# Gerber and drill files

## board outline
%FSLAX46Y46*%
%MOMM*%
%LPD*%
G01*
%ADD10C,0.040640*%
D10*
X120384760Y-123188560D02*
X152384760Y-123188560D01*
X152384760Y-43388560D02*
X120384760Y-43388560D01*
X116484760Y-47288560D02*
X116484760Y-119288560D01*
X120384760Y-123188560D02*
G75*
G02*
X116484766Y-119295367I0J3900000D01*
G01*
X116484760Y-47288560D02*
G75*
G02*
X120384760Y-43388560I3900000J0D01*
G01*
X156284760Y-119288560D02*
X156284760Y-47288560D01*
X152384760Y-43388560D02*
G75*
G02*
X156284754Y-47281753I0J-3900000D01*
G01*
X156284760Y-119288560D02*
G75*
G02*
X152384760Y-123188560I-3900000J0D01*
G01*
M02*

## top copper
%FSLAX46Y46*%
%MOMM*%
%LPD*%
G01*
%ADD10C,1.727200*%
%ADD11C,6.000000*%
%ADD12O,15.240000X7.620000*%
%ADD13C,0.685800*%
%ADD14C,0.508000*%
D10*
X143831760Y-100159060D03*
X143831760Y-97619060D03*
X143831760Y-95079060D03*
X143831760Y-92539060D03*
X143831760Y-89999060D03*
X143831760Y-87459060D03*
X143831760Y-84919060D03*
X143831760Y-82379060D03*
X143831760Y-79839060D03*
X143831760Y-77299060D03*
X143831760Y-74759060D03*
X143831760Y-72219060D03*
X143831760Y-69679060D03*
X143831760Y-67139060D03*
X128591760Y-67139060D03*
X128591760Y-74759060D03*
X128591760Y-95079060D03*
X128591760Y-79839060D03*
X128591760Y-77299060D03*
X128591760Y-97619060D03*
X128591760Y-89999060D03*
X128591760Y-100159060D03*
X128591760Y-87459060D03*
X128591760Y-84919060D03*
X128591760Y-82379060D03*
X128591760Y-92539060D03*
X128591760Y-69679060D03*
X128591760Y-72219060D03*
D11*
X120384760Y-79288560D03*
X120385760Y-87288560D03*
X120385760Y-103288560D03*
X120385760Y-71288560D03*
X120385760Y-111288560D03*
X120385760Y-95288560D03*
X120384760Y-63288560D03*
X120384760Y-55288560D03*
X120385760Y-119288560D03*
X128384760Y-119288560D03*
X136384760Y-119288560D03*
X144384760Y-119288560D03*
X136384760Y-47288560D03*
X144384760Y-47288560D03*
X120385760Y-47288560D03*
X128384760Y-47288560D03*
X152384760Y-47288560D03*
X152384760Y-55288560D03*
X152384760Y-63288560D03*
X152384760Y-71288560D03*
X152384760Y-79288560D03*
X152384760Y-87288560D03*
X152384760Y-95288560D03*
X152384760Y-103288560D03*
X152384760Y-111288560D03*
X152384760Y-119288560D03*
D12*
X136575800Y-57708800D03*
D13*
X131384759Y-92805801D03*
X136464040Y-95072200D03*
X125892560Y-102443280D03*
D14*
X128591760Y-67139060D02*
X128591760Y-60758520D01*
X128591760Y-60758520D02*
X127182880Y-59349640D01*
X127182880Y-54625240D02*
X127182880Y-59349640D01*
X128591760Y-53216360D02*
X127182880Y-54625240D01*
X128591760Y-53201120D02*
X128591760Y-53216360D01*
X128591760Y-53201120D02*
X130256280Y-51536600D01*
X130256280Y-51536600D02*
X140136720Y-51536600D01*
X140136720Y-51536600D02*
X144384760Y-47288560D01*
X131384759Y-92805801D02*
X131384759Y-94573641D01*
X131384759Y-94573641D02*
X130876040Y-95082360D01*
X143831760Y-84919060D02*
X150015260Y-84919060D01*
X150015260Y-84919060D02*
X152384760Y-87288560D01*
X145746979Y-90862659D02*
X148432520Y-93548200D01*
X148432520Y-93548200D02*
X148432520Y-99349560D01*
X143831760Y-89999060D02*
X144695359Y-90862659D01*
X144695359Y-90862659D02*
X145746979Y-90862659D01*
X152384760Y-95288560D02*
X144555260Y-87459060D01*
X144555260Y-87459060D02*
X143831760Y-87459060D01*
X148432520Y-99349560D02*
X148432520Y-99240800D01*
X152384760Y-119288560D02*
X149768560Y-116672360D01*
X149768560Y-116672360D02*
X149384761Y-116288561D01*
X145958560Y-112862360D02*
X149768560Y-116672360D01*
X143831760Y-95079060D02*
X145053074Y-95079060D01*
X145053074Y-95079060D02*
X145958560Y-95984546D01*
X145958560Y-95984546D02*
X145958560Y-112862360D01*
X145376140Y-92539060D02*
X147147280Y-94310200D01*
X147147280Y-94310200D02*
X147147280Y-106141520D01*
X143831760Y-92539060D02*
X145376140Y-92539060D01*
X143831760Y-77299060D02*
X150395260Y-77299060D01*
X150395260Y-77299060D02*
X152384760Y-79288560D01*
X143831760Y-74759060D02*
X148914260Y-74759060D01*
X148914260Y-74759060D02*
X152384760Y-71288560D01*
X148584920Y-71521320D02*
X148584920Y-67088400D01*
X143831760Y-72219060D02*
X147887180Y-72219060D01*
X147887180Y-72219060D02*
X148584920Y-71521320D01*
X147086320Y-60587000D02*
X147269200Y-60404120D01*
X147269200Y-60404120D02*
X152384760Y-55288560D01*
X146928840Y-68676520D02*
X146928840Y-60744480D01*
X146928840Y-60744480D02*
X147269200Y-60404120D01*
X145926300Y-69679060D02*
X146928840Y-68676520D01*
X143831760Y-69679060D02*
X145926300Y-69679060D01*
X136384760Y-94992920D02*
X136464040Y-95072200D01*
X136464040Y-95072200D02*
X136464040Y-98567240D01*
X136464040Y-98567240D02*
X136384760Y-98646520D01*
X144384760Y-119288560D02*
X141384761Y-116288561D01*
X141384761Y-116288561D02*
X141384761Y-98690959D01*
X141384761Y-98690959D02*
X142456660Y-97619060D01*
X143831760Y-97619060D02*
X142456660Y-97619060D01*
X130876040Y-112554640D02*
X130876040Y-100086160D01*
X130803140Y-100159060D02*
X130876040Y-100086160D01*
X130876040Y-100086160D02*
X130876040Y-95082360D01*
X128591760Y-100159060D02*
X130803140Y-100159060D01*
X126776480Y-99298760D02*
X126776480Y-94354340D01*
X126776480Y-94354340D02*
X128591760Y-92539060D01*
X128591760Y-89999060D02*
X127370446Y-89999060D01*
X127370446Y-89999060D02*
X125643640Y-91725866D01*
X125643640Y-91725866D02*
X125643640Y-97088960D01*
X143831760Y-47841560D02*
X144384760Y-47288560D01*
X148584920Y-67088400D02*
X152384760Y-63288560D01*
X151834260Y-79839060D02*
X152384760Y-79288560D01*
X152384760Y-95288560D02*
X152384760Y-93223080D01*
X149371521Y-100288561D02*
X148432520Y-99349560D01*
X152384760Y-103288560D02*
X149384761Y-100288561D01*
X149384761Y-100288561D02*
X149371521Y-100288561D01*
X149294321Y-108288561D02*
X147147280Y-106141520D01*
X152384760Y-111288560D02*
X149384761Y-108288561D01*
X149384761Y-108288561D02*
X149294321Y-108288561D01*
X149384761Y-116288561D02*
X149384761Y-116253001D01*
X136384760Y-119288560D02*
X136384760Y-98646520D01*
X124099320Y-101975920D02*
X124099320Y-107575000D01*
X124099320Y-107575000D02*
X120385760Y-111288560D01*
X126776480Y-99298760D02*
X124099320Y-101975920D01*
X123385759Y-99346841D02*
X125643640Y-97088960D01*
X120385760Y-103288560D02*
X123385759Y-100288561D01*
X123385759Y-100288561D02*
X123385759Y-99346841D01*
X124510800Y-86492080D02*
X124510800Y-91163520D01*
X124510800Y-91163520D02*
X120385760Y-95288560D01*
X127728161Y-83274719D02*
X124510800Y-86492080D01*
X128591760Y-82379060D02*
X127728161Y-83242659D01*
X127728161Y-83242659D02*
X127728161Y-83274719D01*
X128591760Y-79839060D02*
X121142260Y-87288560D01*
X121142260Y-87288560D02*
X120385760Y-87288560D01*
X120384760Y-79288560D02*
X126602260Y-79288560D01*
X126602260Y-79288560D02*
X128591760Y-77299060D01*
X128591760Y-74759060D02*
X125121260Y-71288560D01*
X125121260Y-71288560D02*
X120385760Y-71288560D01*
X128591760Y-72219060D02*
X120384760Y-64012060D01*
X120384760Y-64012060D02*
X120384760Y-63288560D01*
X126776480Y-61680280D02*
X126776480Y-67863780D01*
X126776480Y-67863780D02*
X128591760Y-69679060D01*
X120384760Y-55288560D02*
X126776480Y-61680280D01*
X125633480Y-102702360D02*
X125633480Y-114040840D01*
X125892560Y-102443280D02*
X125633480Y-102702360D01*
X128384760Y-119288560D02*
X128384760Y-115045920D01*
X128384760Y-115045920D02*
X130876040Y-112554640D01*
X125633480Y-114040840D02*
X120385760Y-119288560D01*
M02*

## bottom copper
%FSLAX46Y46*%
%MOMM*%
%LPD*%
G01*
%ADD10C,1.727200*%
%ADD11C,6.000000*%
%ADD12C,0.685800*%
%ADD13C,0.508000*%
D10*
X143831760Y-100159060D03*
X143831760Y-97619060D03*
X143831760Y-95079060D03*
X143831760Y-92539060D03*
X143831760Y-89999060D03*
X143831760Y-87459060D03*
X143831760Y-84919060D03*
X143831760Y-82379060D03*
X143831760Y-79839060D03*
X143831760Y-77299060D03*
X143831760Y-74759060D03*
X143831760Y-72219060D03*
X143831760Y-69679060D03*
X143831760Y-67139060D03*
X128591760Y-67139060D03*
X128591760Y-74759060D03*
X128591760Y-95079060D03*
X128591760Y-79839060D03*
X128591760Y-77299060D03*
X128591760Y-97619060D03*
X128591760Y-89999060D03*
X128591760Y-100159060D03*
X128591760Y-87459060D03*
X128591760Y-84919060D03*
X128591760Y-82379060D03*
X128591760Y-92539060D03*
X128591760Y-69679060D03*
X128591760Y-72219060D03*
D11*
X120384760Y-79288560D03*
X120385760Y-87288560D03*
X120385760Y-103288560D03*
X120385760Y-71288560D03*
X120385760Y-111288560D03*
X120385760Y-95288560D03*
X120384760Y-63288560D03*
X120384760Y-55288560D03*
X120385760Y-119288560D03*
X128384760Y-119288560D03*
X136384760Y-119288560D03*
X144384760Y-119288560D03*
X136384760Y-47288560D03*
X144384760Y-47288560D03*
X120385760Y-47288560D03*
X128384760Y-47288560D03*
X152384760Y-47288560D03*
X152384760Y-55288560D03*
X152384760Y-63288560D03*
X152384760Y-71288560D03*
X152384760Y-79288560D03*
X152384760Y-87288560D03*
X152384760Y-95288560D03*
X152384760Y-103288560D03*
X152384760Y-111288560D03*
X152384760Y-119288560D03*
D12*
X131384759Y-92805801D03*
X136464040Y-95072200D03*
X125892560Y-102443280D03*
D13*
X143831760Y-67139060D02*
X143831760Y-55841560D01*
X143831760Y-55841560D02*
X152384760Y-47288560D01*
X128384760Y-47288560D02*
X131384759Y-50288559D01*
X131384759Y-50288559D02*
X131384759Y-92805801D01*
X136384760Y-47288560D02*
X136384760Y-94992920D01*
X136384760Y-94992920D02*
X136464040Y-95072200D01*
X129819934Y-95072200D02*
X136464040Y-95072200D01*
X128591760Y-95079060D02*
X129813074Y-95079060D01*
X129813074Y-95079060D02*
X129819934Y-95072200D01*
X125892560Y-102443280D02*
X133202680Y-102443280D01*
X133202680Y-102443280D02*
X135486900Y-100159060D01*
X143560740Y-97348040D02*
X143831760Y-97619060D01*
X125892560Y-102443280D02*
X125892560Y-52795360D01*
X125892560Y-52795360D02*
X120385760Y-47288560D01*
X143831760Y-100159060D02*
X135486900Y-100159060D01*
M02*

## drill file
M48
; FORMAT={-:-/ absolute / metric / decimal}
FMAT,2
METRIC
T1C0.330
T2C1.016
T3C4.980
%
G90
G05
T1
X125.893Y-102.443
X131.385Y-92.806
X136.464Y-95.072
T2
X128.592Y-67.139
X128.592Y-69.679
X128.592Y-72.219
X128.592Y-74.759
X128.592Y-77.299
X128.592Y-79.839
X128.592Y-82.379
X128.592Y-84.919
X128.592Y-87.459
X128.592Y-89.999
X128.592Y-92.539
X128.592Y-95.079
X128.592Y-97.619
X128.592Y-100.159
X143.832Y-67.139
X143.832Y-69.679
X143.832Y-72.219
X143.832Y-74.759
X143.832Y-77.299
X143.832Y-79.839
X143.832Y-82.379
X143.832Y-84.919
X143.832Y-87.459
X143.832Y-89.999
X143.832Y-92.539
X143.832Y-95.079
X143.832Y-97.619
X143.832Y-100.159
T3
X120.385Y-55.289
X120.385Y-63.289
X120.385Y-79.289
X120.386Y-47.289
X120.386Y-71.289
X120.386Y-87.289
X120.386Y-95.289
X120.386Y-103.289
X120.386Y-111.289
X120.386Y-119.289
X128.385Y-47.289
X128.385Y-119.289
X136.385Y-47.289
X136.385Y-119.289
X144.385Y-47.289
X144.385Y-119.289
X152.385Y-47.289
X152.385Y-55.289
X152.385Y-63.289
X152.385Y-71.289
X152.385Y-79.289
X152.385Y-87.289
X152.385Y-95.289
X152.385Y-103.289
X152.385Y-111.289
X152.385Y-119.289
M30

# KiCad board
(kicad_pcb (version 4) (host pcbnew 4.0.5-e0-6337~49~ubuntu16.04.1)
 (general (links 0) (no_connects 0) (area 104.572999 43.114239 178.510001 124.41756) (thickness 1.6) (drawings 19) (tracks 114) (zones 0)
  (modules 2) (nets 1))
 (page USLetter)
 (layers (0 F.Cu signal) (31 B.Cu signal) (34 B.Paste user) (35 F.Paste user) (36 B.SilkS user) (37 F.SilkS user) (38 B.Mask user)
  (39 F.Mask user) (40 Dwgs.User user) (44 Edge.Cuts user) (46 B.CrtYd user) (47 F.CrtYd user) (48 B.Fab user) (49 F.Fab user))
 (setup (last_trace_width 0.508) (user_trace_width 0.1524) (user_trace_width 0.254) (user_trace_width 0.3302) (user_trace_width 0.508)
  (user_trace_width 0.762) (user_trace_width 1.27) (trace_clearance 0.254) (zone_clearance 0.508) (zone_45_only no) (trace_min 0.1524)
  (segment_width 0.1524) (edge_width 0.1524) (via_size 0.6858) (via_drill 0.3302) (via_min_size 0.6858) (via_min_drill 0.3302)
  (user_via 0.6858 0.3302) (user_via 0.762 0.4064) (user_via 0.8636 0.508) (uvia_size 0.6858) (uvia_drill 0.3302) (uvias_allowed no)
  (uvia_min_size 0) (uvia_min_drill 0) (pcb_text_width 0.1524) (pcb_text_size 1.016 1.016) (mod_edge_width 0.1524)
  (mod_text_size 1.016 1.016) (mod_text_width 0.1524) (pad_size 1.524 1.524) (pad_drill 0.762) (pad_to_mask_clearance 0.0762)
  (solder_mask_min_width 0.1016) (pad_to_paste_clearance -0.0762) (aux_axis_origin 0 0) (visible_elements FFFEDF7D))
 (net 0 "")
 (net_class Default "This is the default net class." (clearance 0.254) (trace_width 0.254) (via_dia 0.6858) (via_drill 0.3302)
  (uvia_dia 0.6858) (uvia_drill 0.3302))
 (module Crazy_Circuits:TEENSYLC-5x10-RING (layer F.Cu) (at 120.38476 71.28856)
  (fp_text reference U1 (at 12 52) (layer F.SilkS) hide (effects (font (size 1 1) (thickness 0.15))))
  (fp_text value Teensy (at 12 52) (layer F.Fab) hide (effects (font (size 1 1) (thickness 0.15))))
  (fp_line (start 0 51.9) (end 32 51.9) (layer Edge.Cuts) (width 0.04064))
  (fp_line (start 32 -27.9) (end 0 -27.9) (layer Edge.Cuts) (width 0.04064))
  (fp_line (start -3.9 -24) (end -3.9 48) (layer Edge.Cuts) (width 0.04064))
  (fp_arc (start 0 48) (end 0 51.9) (angle 89.9) (layer Edge.Cuts) (width 0.04064))
  (fp_arc (start 0 -24) (end -3.9 -24) (angle 90) (layer Edge.Cuts) (width 0.04064))
  (fp_line (start 35.9 48) (end 35.9 -24) (layer Edge.Cuts) (width 0.04064))
  (fp_arc (start 32 -24) (end 32 -27.9) (angle 89.9) (layer Edge.Cuts) (width 0.04064))
  (fp_arc (start 32 48) (end 35.9 48) (angle 90) (layer Edge.Cuts) (width 0.04064))
  (pad GND thru_hole circle (at 23.447 28.8705 180) (size 1.7272 1.7272) (drill 1.016) (layers *.Cu *.Mask F.SilkS))
  (pad 0 thru_hole circle (at 23.447 26.3305 180) (size 1.7272 1.7272) (drill 1.016) (layers *.Cu *.Mask F.SilkS))
  (pad 1 thru_hole circle (at 23.447 23.7905 180) (size 1.7272 1.7272) (drill 1.016) (layers *.Cu *.Mask F.SilkS))
  (pad 2 thru_hole circle (at 23.447 21.2505 180) (size 1.7272 1.7272) (drill 1.016) (layers *.Cu *.Mask F.SilkS))
  (pad 3 thru_hole circle (at 23.447 18.7105 180) (size 1.7272 1.7272) (drill 1.016) (layers *.Cu *.Mask F.SilkS))
  (pad 4 thru_hole circle (at 23.447 16.1705 180) (size 1.7272 1.7272) (drill 1.016) (layers *.Cu *.Mask F.SilkS))
  (pad 5 thru_hole circle (at 23.447 13.6305 180) (size 1.7272 1.7272) (drill 1.016) (layers *.Cu *.Mask F.SilkS))
  (pad 6 thru_hole circle (at 23.447 11.0905 180) (size 1.7272 1.7272) (drill 1.016) (layers *.Cu *.Mask F.SilkS))
  (pad 7 thru_hole circle (at 23.447 8.5505 180) (size 1.7272 1.7272) (drill 1.016) (layers *.Cu *.Mask F.SilkS))
  (pad 8 thru_hole circle (at 23.447 6.0105 180) (size 1.7272 1.7272) (drill 1.016) (layers *.Cu *.Mask F.SilkS))
  (pad 9 thru_hole circle (at 23.447 3.4705 180) (size 1.7272 1.7272) (drill 1.016) (layers *.Cu *.Mask F.SilkS))
  (pad 10 thru_hole circle (at 23.447 0.9305 180) (size 1.7272 1.7272) (drill 1.016) (layers *.Cu *.Mask F.SilkS))
  (pad 11 thru_hole circle (at 23.447 -1.6095 180) (size 1.7272 1.7272) (drill 1.016) (layers *.Cu *.Mask F.SilkS))
  (pad 12 thru_hole circle (at 23.447 -4.1495 180) (size 1.7272 1.7272) (drill 1.016) (layers *.Cu *.Mask F.SilkS))
  (pad 13 thru_hole circle (at 8.207 -4.1495 180) (size 1.7272 1.7272) (drill 1.016) (layers *.Cu *.Mask F.SilkS))
  (pad 16 thru_hole circle (at 8.207 3.4705 180) (size 1.7272 1.7272) (drill 1.016) (layers *.Cu *.Mask F.SilkS))
  (pad 3.3V thru_hole circle (at 8.207 23.7905 180) (size 1.7272 1.7272) (drill 1.016) (layers *.Cu *.Mask F.SilkS))
  (pad 18 thru_hole circle (at 8.207 8.5505 180) (size 1.7272 1.7272) (drill 1.016) (layers *.Cu *.Mask F.SilkS))
  (pad 17 thru_hole circle (at 8.207 6.0105 180) (size 1.7272 1.7272) (drill 1.016) (layers *.Cu *.Mask F.SilkS))
  (pad G3 thru_hole circle (at 8.207 26.3305 180) (size 1.7272 1.7272) (drill 1.016) (layers *.Cu *.Mask F.SilkS))
  (pad 22 thru_hole circle (at 8.207 18.7105 180) (size 1.7272 1.7272) (drill 1.016) (layers *.Cu *.Mask F.SilkS))
  (pad VIN thru_hole circle (at 8.207 28.8705 180) (size 1.7272 1.7272) (drill 1.016) (layers *.Cu *.Mask F.SilkS))
  (pad 21 thru_hole circle (at 8.207 16.1705 180) (size 1.7272 1.7272) (drill 1.016) (layers *.Cu *.Mask F.SilkS))
  (pad 20 thru_hole circle (at 8.207 13.6305 180) (size 1.7272 1.7272) (drill 1.016) (layers *.Cu *.Mask F.SilkS))
  (pad 19 thru_hole circle (at 8.207 11.0905 180) (size 1.7272 1.7272) (drill 1.016) (layers *.Cu *.Mask F.SilkS))
  (pad 23 thru_hole circle (at 8.207 21.2505 180) (size 1.7272 1.7272) (drill 1.016) (layers *.Cu *.Mask F.SilkS))
  (pad 14 thru_hole circle (at 8.207 -1.6095 180) (size 1.7272 1.7272) (drill 1.016) (layers *.Cu *.Mask F.SilkS))
  (pad 15 thru_hole circle (at 8.207 0.9305 180) (size 1.7272 1.7272) (drill 1.016) (layers *.Cu *.Mask F.SilkS))
  (pad 17 thru_hole circle (at 0 8 90) (size 6 6) (drill 4.98) (layers *.Cu *.Mask))
  (pad 18 thru_hole circle (at 0.001 16 90) (size 6 6) (drill 4.98) (layers *.Cu *.Mask))
  (pad 22 thru_hole circle (at 0.001 32 90) (size 6 6) (drill 4.98) (layers *.Cu *.Mask))
  (pad 16 thru_hole circle (at 0.001 0 90) (size 6 6) (drill 4.98) (layers *.Cu *.Mask))
  (pad 23 thru_hole circle (at 0.001 40 90) (size 6 6) (drill 4.98) (layers *.Cu *.Mask))
  (pad 19 thru_hole circle (at 0.001 24 90) (size 6 6) (drill 4.98) (layers *.Cu *.Mask))
  (pad 15 thru_hole circle (at 0 -8 90) (size 6 6) (drill 4.98) (layers *.Cu *.Mask))
  (pad 14 thru_hole circle (at 0 -16 90) (size 6 6) (drill 4.98) (layers *.Cu *.Mask))
  (pad GND thru_hole circle (at 0.001 48 90) (size 6 6) (drill 4.98) (layers *.Cu *.Mask))
  (pad VIN thru_hole circle (at 8 48 90) (size 6 6) (drill 4.98) (layers *.Cu *.Mask))
  (pad 3.3V thru_hole circle (at 16 48 90) (size 6 6) (drill 4.98) (layers *.Cu *.Mask))
  (pad 0/TX thru_hole circle (at 24 48 90) (size 6 6) (drill 4.98) (layers *.Cu *.Mask))
  (pad 3.3V thru_hole circle (at 16 -24 90) (size 6 6) (drill 4.98) (layers *.Cu *.Mask))
  (pad 13 thru_hole circle (at 24 -24 90) (size 6 6) (drill 4.98) (layers *.Cu *.Mask))
  (pad GND thru_hole circle (at 0.001 -24 90) (size 6 6) (drill 4.98) (layers *.Cu *.Mask))
  (pad VIN thru_hole circle (at 8 -24 90) (size 6 6) (drill 4.98) (layers *.Cu *.Mask))
  (pad 12 thru_hole circle (at 32 -24 90) (size 6 6) (drill 4.98) (layers *.Cu *.Mask))
  (pad 11 thru_hole circle (at 32 -16 90) (size 6 6) (drill 4.98) (layers *.Cu *.Mask))
  (pad 10 thru_hole circle (at 32 -8 90) (size 6 6) (drill 4.98) (layers *.Cu *.Mask))
  (pad 9 thru_hole circle (at 32 0 90) (size 6 6) (drill 4.98) (layers *.Cu *.Mask))
  (pad 8 thru_hole circle (at 32 8 90) (size 6 6) (drill 4.98) (layers *.Cu *.Mask))
  (pad 5 thru_hole circle (at 32 16 90) (size 6 6) (drill 4.98) (layers *.Cu *.Mask))
  (pad 4 thru_hole circle (at 32 24 90) (size 6 6) (drill 4.98) (layers *.Cu *.Mask))
  (pad 3 thru_hole circle (at 32 32 90) (size 6 6) (drill 4.98) (layers *.Cu *.Mask))
  (pad 2 thru_hole circle (at 32 40 90) (size 6 6) (drill 4.98) (layers *.Cu *.Mask))
  (pad 1/RX thru_hole circle (at 32 48 90) (size 6 6) (drill 4.98) (layers *.Cu *.Mask)))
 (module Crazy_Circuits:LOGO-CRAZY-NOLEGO (layer F.Cu) (at 136.5758 61.6458)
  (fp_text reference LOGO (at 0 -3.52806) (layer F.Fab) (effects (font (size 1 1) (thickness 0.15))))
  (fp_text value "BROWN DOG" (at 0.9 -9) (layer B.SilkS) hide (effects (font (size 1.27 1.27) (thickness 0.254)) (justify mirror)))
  (pad BG smd oval (at 0 -3.937) (size 15.24 7.62) (layers F.Cu)))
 (segment (start 128.59176 67.13906) (end 128.59176 60.75852) (width 0.508) (layer F.Cu) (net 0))
 (segment (start 128.59176 60.75852) (end 127.18288 59.34964) (width 0.508) (layer F.Cu) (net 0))
 (segment (start 127.18288 54.62524) (end 127.18288 59.34964) (width 0.508) (layer F.Cu) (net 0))
 (segment (start 128.59176 53.21636) (end 127.18288 54.62524) (width 0.508) (layer F.Cu) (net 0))
 (segment (start 128.59176 53.20112) (end 128.59176 53.21636) (width 0.508) (layer F.Cu) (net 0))
 (segment (start 128.59176 53.20112) (end 130.25628 51.5366) (width 0.508) (layer F.Cu) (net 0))
 (segment (start 130.25628 51.5366) (end 140.13672 51.5366) (width 0.508) (layer F.Cu) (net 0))
 (segment (start 140.13672 51.5366) (end 144.38476 47.28856) (width 0.508) (layer F.Cu) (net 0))
 (segment (start 143.83176 67.13906) (end 143.83176 55.84156) (width 0.508) (layer B.Cu) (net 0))
 (segment (start 143.83176 55.84156) (end 152.38476 47.28856) (width 0.508) (layer B.Cu) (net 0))
 (segment (start 131.384759 92.805801) (end 131.384759 94.573641) (width 0.508) (layer F.Cu) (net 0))
 (segment (start 131.384759 94.573641) (end 130.87604 95.08236) (width 0.508) (layer F.Cu) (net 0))
 (via (at 131.384759 92.805801) (size 0.6858) (drill 0.3302) (layers F.Cu B.Cu) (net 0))
 (segment (start 128.38476 47.28856) (end 131.384759 50.288559) (width 0.508) (layer B.Cu) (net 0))
 (segment (start 131.384759 50.288559) (end 131.384759 92.805801) (width 0.508) (layer B.Cu) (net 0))
 (segment (start 136.38476 47.28856) (end 136.38476 94.99292) (width 0.508) (layer B.Cu) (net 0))
 (segment (start 136.38476 94.99292) (end 136.46404 95.0722) (width 0.508) (layer B.Cu) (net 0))
 (segment (start 143.83176 84.91906) (end 150.01526 84.91906) (width 0.508) (layer F.Cu) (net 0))
 (segment (start 150.01526 84.91906) (end 152.38476 87.28856) (width 0.508) (layer F.Cu) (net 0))
 (segment (start 145.746979 90.862659) (end 148.43252 93.5482) (width 0.508) (layer F.Cu) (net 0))
 (segment (start 148.43252 93.5482) (end 148.43252 99.34956) (width 0.508) (layer F.Cu) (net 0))
 (segment (start 143.83176 89.99906) (end 144.695359 90.862659) (width 0.508) (layer F.Cu) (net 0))
 (segment (start 144.695359 90.862659) (end 145.746979 90.862659) (width 0.508) (layer F.Cu) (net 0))
 (segment (start 152.38476 95.28856) (end 144.55526 87.45906) (width 0.508) (layer F.Cu) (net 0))
 (segment (start 144.55526 87.45906) (end 143.83176 87.45906) (width 0.508) (layer F.Cu) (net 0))
 (segment (start 148.43252 99.34956) (end 148.43252 99.2408) (width 0.508) (layer F.Cu) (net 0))
 (segment (start 152.38476 119.28856) (end 149.76856 116.67236) (width 0.508) (layer F.Cu) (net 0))
 (segment (start 149.76856 116.67236) (end 149.384761 116.288561) (width 0.508) (layer F.Cu) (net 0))
 (segment (start 145.95856 112.86236) (end 149.76856 116.67236) (width 0.508) (layer F.Cu) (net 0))
 (segment (start 143.83176 95.07906) (end 145.053074 95.07906) (width 0.508) (layer F.Cu) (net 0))
 (segment (start 145.053074 95.07906) (end 145.95856 95.984546) (width 0.508) (layer F.Cu) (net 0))
 (segment (start 145.95856 95.984546) (end 145.95856 112.86236) (width 0.508) (layer F.Cu) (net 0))
 (segment (start 145.37614 92.53906) (end 147.14728 94.3102) (width 0.508) (layer F.Cu) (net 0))
 (segment (start 147.14728 94.3102) (end 147.14728 106.14152) (width 0.508) (layer F.Cu) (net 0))
 (segment (start 143.83176 92.53906) (end 145.37614 92.53906) (width 0.508) (layer F.Cu) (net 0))
 (segment (start 143.83176 77.29906) (end 150.39526 77.29906) (width 0.508) (layer F.Cu) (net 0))
 (segment (start 150.39526 77.29906) (end 152.38476 79.28856) (width 0.508) (layer F.Cu) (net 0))
 (segment (start 143.83176 74.75906) (end 148.91426 74.75906) (width 0.508) (layer F.Cu) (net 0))
 (segment (start 148.91426 74.75906) (end 152.38476 71.28856) (width 0.508) (layer F.Cu) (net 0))
 (segment (start 148.58492 71.52132) (end 148.58492 67.0884) (width 0.508) (layer F.Cu) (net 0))
 (segment (start 143.83176 72.21906) (end 147.88718 72.21906) (width 0.508) (layer F.Cu) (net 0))
 (segment (start 147.88718 72.21906) (end 148.58492 71.52132) (width 0.508) (layer F.Cu) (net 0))
 (segment (start 147.08632 60.587) (end 147.2692 60.40412) (width 0.508) (layer F.Cu) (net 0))
 (segment (start 147.2692 60.40412) (end 152.38476 55.28856) (width 0.508) (layer F.Cu) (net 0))
 (segment (start 146.92884 68.67652) (end 146.92884 60.74448) (width 0.508) (layer F.Cu) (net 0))
 (segment (start 146.92884 60.74448) (end 147.2692 60.40412) (width 0.508) (layer F.Cu) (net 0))
 (segment (start 145.9263 69.67906) (end 146.92884 68.67652) (width 0.508) (layer F.Cu) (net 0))
 (segment (start 143.83176 69.67906) (end 145.9263 69.67906) (width 0.508) (layer F.Cu) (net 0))
 (segment (start 136.38476 94.99292) (end 136.46404 95.0722) (width 0.508) (layer F.Cu) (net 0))
 (segment (start 136.46404 95.0722) (end 136.46404 98.56724) (width 0.508) (layer F.Cu) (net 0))
 (segment (start 136.46404 98.56724) (end 136.38476 98.64652) (width 0.508) (layer F.Cu) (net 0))
 (segment (start 129.819934 95.0722) (end 136.46404 95.0722) (width 0.508) (layer B.Cu) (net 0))
 (via (at 136.46404 95.0722) (size 0.6858) (drill 0.3302) (layers F.Cu B.Cu) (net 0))
 (segment (start 128.59176 95.07906) (end 129.813074 95.07906) (width 0.508) (layer B.Cu) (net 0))
 (segment (start 129.813074 95.07906) (end 129.819934 95.0722) (width 0.508) (layer B.Cu) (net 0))
 (segment (start 144.38476 119.28856) (end 141.384761 116.288561) (width 0.508) (layer F.Cu) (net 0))
 (segment (start 141.384761 116.288561) (end 141.384761 98.690959) (width 0.508) (layer F.Cu) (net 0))
 (segment (start 141.384761 98.690959) (end 142.45666 97.61906) (width 0.508) (layer F.Cu) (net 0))
 (segment (start 143.83176 97.61906) (end 142.45666 97.61906) (width 0.508) (layer F.Cu) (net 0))
 (segment (start 125.89256 102.44328) (end 133.20268 102.44328) (width 0.508) (layer B.Cu) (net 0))
 (segment (start 133.20268 102.44328) (end 135.4869 100.15906) (width 0.508) (layer B.Cu) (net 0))
 (segment (start 130.87604 112.55464) (end 130.87604 100.08616) (width 0.508) (layer F.Cu) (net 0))
 (segment (start 130.80314 100.15906) (end 130.87604 100.08616) (width 0.508) (layer F.Cu) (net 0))
 (segment (start 130.87604 100.08616) (end 130.87604 95.08236) (width 0.508) (layer F.Cu) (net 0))
 (segment (start 128.59176 100.15906) (end 130.80314 100.15906) (width 0.508) (layer F.Cu) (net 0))
 (segment (start 126.77648 99.29876) (end 126.77648 94.35434) (width 0.508) (layer F.Cu) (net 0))
 (segment (start 126.77648 94.35434) (end 128.59176 92.53906) (width 0.508) (layer F.Cu) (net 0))
 (segment (start 128.59176 89.99906) (end 127.370446 89.99906) (width 0.508) (layer F.Cu) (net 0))
 (segment (start 127.370446 89.99906) (end 125.64364 91.725866) (width 0.508) (layer F.Cu) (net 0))
 (segment (start 125.64364 91.725866) (end 125.64364 97.08896) (width 0.508) (layer F.Cu) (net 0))
 (segment (start 143.83176 47.84156) (end 144.38476 47.28856) (width 0.508) (layer F.Cu) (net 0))
 (segment (start 148.58492 67.0884) (end 152.38476 63.28856) (width 0.508) (layer F.Cu) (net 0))
 (segment (start 151.83426 79.83906) (end 152.38476 79.28856) (width 0.508) (layer F.Cu) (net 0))
 (segment (start 152.38476 95.28856) (end 152.38476 93.22308) (width 0.508) (layer F.Cu) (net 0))
 (segment (start 149.371521 100.288561) (end 148.43252 99.34956) (width 0.508) (layer F.Cu) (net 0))
 (segment (start 152.38476 103.28856) (end 149.384761 100.288561) (width 0.508) (layer F.Cu) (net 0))
 (segment (start 149.384761 100.288561) (end 149.371521 100.288561) (width 0.508) (layer F.Cu) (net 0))
 (segment (start 149.294321 108.288561) (end 147.14728 106.14152) (width 0.508) (layer F.Cu) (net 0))
 (segment (start 152.38476 111.28856) (end 149.384761 108.288561) (width 0.508) (layer F.Cu) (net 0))
 (segment (start 149.384761 108.288561) (end 149.294321 108.288561) (width 0.508) (layer F.Cu) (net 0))
 (segment (start 149.384761 116.288561) (end 149.384761 116.253001) (width 0.508) (layer F.Cu) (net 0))
 (segment (start 143.56074 97.34804) (end 143.83176 97.61906) (width 0.508) (layer B.Cu) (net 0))
 (segment (start 136.38476 119.28856) (end 136.38476 98.64652) (width 0.508) (layer F.Cu) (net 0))
 (segment (start 124.09932 101.97592) (end 124.09932 107.575) (width 0.508) (layer F.Cu) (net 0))
 (segment (start 124.09932 107.575) (end 120.38576 111.28856) (width 0.508) (layer F.Cu) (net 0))
 (segment (start 126.77648 99.29876) (end 124.09932 101.97592) (width 0.508) (layer F.Cu) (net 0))
 (segment (start 123.385759 99.346841) (end 125.64364 97.08896) (width 0.508) (layer F.Cu) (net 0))
 (segment (start 120.38576 103.28856) (end 123.385759 100.288561) (width 0.508) (layer F.Cu) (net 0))
 (segment (start 123.385759 100.288561) (end 123.385759 99.346841) (width 0.508) (layer F.Cu) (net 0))
 (segment (start 124.5108 86.49208) (end 124.5108 91.16352) (width 0.508) (layer F.Cu) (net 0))
 (segment (start 124.5108 91.16352) (end 120.38576 95.28856) (width 0.508) (layer F.Cu) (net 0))
 (segment (start 127.728161 83.274719) (end 124.5108 86.49208) (width 0.508) (layer F.Cu) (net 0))
 (segment (start 128.59176 82.37906) (end 127.728161 83.242659) (width 0.508) (layer F.Cu) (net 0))
 (segment (start 127.728161 83.242659) (end 127.728161 83.274719) (width 0.508) (layer F.Cu) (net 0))
 (segment (start 128.59176 79.83906) (end 121.14226 87.28856) (width 0.508) (layer F.Cu) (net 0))
 (segment (start 121.14226 87.28856) (end 120.38576 87.28856) (width 0.508) (layer F.Cu) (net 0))
 (segment (start 120.38476 79.28856) (end 126.60226 79.28856) (width 0.508) (layer F.Cu) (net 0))
 (segment (start 126.60226 79.28856) (end 128.59176 77.29906) (width 0.508) (layer F.Cu) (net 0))
 (segment (start 128.59176 74.75906) (end 125.12126 71.28856) (width 0.508) (layer F.Cu) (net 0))
 (segment (start 125.12126 71.28856) (end 120.38576 71.28856) (width 0.508) (layer F.Cu) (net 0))
 (segment (start 128.59176 72.21906) (end 120.38476 64.01206) (width 0.508) (layer F.Cu) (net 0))
 (segment (start 120.38476 64.01206) (end 120.38476 63.28856) (width 0.508) (layer F.Cu) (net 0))
 (segment (start 126.77648 61.68028) (end 126.77648 67.86378) (width 0.508) (layer F.Cu) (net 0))
 (segment (start 126.77648 67.86378) (end 128.59176 69.67906) (width 0.508) (layer F.Cu) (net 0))
 (segment (start 120.38476 55.28856) (end 126.77648 61.68028) (width 0.508) (layer F.Cu) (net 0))
 (segment (start 125.89256 102.44328) (end 125.89256 52.79536) (width 0.508) (layer B.Cu) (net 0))
 (segment (start 125.89256 52.79536) (end 120.38576 47.28856) (width 0.508) (layer B.Cu) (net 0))
 (via (at 125.89256 102.44328) (size 0.6858) (drill 0.3302) (layers F.Cu B.Cu) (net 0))
 (segment (start 125.63348 102.70236) (end 125.63348 114.04084) (width 0.508) (layer F.Cu) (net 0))
 (segment (start 125.89256 102.44328) (end 125.63348 102.70236) (width 0.508) (layer F.Cu) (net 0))
 (segment (start 143.83176 100.15906) (end 135.4869 100.15906) (width 0.508) (layer B.Cu) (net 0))
 (segment (start 128.38476 119.28856) (end 128.38476 115.04592) (width 0.508) (layer F.Cu) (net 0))
 (segment (start 128.38476 115.04592) (end 130.87604 112.55464) (width 0.508) (layer F.Cu) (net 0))
 (segment (start 125.63348 114.04084) (end 120.38576 119.28856) (width 0.508) (layer F.Cu) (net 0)))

